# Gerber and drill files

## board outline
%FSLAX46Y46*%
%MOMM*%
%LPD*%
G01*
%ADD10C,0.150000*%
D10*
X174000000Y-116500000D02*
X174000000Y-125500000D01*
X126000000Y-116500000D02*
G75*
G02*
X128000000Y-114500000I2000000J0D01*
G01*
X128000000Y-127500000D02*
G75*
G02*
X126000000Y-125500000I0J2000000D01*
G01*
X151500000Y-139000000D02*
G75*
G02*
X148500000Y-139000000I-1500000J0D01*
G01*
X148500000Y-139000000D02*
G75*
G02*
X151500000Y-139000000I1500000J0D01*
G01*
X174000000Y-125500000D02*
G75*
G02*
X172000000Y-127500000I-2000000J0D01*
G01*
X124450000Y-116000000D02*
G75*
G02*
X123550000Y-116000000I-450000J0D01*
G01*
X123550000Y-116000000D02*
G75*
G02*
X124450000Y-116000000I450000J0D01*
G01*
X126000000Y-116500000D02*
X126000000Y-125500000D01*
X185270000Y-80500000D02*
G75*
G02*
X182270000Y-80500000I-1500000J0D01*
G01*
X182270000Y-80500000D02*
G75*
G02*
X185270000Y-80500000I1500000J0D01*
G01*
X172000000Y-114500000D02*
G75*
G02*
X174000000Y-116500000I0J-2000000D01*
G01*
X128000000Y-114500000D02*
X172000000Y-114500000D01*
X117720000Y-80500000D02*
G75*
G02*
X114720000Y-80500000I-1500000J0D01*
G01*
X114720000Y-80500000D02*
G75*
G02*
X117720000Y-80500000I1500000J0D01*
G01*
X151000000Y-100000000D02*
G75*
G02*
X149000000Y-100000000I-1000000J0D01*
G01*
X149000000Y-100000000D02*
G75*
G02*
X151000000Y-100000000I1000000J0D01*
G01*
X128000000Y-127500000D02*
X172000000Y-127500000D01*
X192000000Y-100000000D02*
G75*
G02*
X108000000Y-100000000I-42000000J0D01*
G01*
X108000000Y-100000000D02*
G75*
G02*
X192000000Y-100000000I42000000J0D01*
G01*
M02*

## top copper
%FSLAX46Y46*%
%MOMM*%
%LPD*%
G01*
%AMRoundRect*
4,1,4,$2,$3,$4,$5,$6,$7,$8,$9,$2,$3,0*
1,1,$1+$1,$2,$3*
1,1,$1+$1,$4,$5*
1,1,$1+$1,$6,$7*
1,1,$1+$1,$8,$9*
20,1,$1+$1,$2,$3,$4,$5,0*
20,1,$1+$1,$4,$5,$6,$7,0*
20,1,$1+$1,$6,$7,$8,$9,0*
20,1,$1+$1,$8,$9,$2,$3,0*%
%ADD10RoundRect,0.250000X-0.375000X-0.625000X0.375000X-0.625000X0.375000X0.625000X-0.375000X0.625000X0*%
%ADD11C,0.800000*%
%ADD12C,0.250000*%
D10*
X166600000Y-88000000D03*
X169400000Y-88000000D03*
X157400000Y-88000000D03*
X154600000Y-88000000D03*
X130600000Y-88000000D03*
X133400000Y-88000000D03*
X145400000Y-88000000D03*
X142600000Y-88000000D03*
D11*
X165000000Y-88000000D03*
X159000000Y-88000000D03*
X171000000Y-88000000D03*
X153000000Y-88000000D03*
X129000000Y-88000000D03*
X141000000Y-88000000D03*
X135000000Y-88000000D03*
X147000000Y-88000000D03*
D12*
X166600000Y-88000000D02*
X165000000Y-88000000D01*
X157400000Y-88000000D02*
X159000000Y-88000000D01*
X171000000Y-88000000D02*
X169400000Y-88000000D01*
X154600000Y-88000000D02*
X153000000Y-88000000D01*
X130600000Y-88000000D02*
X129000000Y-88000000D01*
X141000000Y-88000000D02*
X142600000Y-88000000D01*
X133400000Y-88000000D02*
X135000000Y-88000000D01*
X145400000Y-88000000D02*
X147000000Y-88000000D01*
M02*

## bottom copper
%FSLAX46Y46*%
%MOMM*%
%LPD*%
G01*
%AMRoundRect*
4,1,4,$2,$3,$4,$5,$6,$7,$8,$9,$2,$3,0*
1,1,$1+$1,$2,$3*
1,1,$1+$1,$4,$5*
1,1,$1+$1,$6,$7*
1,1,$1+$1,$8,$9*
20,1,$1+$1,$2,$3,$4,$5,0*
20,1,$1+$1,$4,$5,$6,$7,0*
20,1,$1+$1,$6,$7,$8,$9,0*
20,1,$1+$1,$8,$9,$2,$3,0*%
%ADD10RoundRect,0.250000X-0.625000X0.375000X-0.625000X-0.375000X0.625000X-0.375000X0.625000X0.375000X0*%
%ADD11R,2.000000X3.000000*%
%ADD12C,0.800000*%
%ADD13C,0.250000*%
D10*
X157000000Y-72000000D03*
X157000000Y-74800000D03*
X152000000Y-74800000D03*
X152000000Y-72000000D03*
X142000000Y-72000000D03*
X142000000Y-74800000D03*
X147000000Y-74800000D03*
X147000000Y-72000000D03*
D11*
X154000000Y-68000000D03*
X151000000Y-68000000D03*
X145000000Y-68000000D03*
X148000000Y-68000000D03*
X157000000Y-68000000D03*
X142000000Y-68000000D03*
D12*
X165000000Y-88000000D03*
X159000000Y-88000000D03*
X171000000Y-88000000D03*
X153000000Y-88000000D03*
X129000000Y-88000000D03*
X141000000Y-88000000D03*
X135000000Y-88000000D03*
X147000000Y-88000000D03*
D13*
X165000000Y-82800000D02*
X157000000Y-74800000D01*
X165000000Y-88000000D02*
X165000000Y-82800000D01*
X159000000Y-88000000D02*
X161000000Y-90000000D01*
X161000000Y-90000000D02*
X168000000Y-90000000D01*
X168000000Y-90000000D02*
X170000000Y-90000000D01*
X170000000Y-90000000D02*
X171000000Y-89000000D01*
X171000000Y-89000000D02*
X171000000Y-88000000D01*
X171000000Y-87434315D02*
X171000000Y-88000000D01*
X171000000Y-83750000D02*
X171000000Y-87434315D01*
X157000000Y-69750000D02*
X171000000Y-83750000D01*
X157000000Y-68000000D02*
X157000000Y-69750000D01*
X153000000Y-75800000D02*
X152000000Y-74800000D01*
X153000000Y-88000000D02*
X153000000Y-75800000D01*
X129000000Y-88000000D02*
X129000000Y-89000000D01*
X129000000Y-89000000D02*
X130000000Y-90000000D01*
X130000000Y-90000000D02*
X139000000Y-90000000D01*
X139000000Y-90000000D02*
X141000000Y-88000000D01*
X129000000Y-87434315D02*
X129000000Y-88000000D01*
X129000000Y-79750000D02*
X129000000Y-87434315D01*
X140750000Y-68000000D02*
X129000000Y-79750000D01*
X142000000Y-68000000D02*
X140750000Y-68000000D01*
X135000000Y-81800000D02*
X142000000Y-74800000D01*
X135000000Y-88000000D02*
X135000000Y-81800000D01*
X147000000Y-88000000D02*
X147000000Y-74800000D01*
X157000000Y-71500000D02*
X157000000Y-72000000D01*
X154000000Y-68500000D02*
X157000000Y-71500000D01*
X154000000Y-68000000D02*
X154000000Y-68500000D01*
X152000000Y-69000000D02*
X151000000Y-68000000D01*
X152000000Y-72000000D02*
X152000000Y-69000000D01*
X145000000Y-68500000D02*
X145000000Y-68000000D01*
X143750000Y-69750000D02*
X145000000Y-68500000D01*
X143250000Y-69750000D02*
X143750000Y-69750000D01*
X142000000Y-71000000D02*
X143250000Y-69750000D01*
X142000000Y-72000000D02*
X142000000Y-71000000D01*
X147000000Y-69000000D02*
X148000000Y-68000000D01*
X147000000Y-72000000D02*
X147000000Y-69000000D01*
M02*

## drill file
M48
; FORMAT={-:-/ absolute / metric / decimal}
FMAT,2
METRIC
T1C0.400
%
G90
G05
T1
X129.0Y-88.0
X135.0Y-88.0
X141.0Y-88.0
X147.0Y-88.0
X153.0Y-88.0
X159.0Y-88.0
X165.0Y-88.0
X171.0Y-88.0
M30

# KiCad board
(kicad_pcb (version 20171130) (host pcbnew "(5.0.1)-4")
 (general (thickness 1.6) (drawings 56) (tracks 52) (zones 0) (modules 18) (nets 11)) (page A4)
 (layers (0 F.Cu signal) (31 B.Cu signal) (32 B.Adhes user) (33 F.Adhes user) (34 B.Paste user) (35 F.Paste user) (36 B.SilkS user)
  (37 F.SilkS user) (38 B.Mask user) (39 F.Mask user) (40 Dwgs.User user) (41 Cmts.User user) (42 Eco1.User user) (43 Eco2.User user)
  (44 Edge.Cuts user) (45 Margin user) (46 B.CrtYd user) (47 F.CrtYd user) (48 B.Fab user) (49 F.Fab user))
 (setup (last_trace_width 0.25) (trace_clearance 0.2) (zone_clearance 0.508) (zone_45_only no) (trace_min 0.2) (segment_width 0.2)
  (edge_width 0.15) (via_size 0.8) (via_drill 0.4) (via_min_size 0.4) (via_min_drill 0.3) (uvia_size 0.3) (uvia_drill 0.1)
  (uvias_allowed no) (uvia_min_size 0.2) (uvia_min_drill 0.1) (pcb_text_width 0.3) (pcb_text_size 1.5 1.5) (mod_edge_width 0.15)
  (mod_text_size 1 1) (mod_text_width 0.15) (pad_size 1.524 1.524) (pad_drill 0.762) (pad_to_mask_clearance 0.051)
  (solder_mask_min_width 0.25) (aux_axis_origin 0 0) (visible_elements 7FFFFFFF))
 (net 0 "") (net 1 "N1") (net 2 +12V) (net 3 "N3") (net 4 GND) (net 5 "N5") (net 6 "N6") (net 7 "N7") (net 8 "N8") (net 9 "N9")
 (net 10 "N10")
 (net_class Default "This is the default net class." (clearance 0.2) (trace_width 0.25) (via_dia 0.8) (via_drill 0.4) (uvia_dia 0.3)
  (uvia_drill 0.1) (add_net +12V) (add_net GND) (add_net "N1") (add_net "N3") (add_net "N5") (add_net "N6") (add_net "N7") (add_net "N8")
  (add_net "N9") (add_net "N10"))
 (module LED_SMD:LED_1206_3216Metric (layer F.Cu) (at 168 88)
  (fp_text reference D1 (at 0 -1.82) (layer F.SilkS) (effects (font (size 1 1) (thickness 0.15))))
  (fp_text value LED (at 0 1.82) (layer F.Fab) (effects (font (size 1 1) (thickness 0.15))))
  (pad 1 smd roundrect (at -1.4 0) (size 1.25 1.75) (layers F.Cu F.Paste F.Mask) (roundrect_rratio 0.2) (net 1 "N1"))
  (pad 2 smd roundrect (at 1.4 0) (size 1.25 1.75) (layers F.Cu F.Paste F.Mask) (roundrect_rratio 0.2) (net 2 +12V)))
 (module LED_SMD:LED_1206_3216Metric (layer F.Cu) (at 156 88)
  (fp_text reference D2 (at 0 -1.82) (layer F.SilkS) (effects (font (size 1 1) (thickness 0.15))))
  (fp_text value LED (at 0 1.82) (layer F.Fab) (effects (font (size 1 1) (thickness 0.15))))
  (pad 2 smd roundrect (at 1.4 0) (size 1.25 1.75) (layers F.Cu F.Paste F.Mask) (roundrect_rratio 0.2) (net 2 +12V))
  (pad 1 smd roundrect (at -1.4 0) (size 1.25 1.75) (layers F.Cu F.Paste F.Mask) (roundrect_rratio 0.2) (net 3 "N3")))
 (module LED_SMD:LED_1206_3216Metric (layer F.Cu) (at 132 88)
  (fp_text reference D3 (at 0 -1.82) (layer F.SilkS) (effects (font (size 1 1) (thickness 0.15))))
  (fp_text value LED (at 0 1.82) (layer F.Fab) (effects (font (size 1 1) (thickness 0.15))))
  (pad 1 smd roundrect (at -1.4 0) (size 1.25 1.75) (layers F.Cu F.Paste F.Mask) (roundrect_rratio 0.2) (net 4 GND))
  (pad 2 smd roundrect (at 1.4 0) (size 1.25 1.75) (layers F.Cu F.Paste F.Mask) (roundrect_rratio 0.2) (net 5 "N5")))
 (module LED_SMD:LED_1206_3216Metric (layer F.Cu) (at 144 88)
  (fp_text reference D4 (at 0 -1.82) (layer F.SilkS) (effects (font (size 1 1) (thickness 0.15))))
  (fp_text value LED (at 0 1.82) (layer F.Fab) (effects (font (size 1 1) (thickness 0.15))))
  (pad 2 smd roundrect (at 1.4 0) (size 1.25 1.75) (layers F.Cu F.Paste F.Mask) (roundrect_rratio 0.2) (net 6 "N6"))
  (pad 1 smd roundrect (at -1.4 0) (size 1.25 1.75) (layers F.Cu F.Paste F.Mask) (roundrect_rratio 0.2) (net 4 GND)))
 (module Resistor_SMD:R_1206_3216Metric (layer B.Cu) (at 157 73.4 270)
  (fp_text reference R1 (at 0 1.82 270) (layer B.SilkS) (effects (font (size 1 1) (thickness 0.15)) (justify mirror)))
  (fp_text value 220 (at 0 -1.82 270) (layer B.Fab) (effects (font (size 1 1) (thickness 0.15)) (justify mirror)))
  (pad 1 smd roundrect (at -1.4 0 270) (size 1.25 1.75) (layers B.Cu B.Paste B.Mask) (roundrect_rratio 0.2) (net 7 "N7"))
  (pad 2 smd roundrect (at 1.4 0 270) (size 1.25 1.75) (layers B.Cu B.Paste B.Mask) (roundrect_rratio 0.2) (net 1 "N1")))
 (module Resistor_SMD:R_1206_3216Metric (layer B.Cu) (at 152 73.4 270)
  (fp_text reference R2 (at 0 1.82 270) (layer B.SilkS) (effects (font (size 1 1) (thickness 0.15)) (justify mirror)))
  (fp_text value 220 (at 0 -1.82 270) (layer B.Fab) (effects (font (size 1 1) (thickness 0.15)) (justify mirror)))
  (pad 2 smd roundrect (at 1.4 0 270) (size 1.25 1.75) (layers B.Cu B.Paste B.Mask) (roundrect_rratio 0.2) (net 3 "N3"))
  (pad 1 smd roundrect (at -1.4 0 270) (size 1.25 1.75) (layers B.Cu B.Paste B.Mask) (roundrect_rratio 0.2) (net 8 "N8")))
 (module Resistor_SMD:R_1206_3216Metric (layer B.Cu) (at 142 73.4 270)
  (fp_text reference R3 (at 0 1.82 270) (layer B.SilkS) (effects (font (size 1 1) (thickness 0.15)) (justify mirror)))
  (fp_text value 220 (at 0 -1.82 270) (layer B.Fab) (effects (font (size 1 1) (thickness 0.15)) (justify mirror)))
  (pad 1 smd roundrect (at -1.4 0 270) (size 1.25 1.75) (layers B.Cu B.Paste B.Mask) (roundrect_rratio 0.2) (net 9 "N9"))
  (pad 2 smd roundrect (at 1.4 0 270) (size 1.25 1.75) (layers B.Cu B.Paste B.Mask) (roundrect_rratio 0.2) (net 5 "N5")))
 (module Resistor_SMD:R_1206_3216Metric (layer B.Cu) (at 147 73.4 270)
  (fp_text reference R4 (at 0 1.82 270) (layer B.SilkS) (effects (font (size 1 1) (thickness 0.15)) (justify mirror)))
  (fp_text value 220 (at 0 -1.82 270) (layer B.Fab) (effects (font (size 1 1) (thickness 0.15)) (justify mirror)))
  (pad 2 smd roundrect (at 1.4 0 270) (size 1.25 1.75) (layers B.Cu B.Paste B.Mask) (roundrect_rratio 0.2) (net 6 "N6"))
  (pad 1 smd roundrect (at -1.4 0 270) (size 1.25 1.75) (layers B.Cu B.Paste B.Mask) (roundrect_rratio 0.2) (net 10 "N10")))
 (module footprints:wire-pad (layer B.Cu) (at 154 66)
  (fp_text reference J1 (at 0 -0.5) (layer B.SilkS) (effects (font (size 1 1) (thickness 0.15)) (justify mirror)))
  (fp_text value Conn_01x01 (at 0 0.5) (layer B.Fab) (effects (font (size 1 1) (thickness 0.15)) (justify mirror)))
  (pad 1 smd rect (at 0 2) (size 2 3) (layers B.Cu B.Paste B.Mask) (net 7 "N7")))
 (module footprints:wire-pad (layer B.Cu) (at 151 66)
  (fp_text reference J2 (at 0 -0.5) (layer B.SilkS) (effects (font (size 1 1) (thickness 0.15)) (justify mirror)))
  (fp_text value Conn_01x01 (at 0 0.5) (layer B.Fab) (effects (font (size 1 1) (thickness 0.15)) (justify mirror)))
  (pad 1 smd rect (at 0 2) (size 2 3) (layers B.Cu B.Paste B.Mask) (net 8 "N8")))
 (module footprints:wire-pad (layer B.Cu) (at 145 66)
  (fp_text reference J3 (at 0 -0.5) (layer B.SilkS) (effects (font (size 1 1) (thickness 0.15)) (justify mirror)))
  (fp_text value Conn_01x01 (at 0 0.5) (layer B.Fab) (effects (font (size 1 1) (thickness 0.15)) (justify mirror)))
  (pad 1 smd rect (at 0 2) (size 2 3) (layers B.Cu B.Paste B.Mask) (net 9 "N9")))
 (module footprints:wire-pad (layer B.Cu) (at 148 66)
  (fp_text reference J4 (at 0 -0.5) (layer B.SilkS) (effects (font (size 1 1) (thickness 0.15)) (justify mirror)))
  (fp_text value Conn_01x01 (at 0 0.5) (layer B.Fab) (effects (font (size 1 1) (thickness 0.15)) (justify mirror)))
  (pad 1 smd rect (at 0 2) (size 2 3) (layers B.Cu B.Paste B.Mask) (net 10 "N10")))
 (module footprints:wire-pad (layer B.Cu) (at 157 66)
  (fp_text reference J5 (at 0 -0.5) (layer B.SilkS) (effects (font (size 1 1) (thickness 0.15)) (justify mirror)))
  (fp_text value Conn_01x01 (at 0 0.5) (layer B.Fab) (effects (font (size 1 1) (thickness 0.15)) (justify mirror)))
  (pad 1 smd rect (at 0 2) (size 2 3) (layers B.Cu B.Paste B.Mask) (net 2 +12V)))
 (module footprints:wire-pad (layer B.Cu) (at 142 66)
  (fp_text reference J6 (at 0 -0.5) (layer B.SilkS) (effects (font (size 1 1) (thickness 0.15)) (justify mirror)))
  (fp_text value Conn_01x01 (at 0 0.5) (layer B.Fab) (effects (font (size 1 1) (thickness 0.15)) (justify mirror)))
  (pad 1 smd rect (at 0 2) (size 2 3) (layers B.Cu B.Paste B.Mask) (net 4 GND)))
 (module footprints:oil (layer F.Cu) (at 168 92)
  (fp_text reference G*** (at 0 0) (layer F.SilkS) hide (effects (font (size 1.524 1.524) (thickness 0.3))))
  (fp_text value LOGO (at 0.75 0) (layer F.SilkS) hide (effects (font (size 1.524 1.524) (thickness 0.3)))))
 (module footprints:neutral (layer F.Cu) (at 156 92)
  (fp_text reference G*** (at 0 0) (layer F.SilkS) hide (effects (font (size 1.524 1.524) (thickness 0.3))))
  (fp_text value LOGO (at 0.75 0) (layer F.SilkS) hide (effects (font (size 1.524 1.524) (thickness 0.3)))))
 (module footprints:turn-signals (layer F.Cu) (at 144 92)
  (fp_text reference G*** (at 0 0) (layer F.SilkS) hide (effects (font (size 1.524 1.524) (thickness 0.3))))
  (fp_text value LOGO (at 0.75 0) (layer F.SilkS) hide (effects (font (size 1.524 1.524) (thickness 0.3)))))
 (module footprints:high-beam (layer F.Cu) (at 132 92)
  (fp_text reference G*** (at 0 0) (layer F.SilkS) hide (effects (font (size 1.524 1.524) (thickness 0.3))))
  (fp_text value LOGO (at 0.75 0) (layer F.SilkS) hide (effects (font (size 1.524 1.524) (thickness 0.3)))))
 (gr_line (start 174 116.5) (end 174 125.5) (layer Edge.Cuts) (width 0.15))
 (gr_arc (start 128 116.5) (end 128 114.5) (angle -90) (layer Edge.Cuts) (width 0.15))
 (gr_arc (start 128 125.5) (end 126 125.5) (angle -90) (layer Edge.Cuts) (width 0.15))
 (gr_circle (center 150 139) (end 151.5 139) (layer Edge.Cuts) (width 0.15))
 (gr_arc (start 172 125.5) (end 172 127.5) (angle -90) (layer Edge.Cuts) (width 0.15))
 (gr_circle (center 124 116) (end 124.45 116) (layer Edge.Cuts) (width 0.15))
 (gr_line (start 126 116.5) (end 126 125.5) (layer Edge.Cuts) (width 0.15))
 (gr_circle (center 183.77 80.5) (end 185.27 80.5) (layer Edge.Cuts) (width 0.15))
 (gr_arc (start 172 116.5) (end 174 116.5) (angle -90) (layer Edge.Cuts) (width 0.15))
 (gr_line (start 128 114.5) (end 172 114.5) (layer Edge.Cuts) (width 0.15))
 (gr_circle (center 116.22 80.5) (end 117.72 80.5) (layer Edge.Cuts) (width 0.15))
 (gr_circle (center 150 100) (end 151 100) (layer Edge.Cuts) (width 0.15))
 (gr_line (start 128 127.5) (end 172 127.5) (layer Edge.Cuts) (width 0.15))
 (gr_circle (center 150 100) (end 192 100) (layer Edge.Cuts) (width 0.15))
 (via (at 165 88) (size 0.8) (drill 0.4) (layers F.Cu B.Cu) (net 1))
 (segment (start 166.6 88) (end 165 88) (width 0.25) (layer F.Cu) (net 1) (status 10))
 (segment (start 165 82.8) (end 157 74.8) (width 0.25) (layer B.Cu) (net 1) (status 20))
 (segment (start 165 88) (end 165 82.8) (width 0.25) (layer B.Cu) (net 1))
 (via (at 159 88) (size 0.8) (drill 0.4) (layers F.Cu B.Cu) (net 2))
 (segment (start 157.4 88) (end 159 88) (width 0.25) (layer F.Cu) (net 2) (status 10))
 (segment (start 159 88) (end 161 90) (width 0.25) (layer B.Cu) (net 2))
 (segment (start 161 90) (end 168 90) (width 0.25) (layer B.Cu) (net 2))
 (segment (start 168 90) (end 170 90) (width 0.25) (layer B.Cu) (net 2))
 (segment (start 170 90) (end 171 89) (width 0.25) (layer B.Cu) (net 2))
 (via (at 171 88) (size 0.8) (drill 0.4) (layers F.Cu B.Cu) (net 2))
 (segment (start 171 89) (end 171 88) (width 0.25) (layer B.Cu) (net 2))
 (segment (start 171 88) (end 169.4 88) (width 0.25) (layer F.Cu) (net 2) (status 20))
 (segment (start 171 87.434315) (end 171 88) (width 0.25) (layer B.Cu) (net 2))
 (segment (start 171 83.75) (end 171 87.434315) (width 0.25) (layer B.Cu) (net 2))
 (segment (start 157 69.75) (end 171 83.75) (width 0.25) (layer B.Cu) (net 2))
 (segment (start 157 68) (end 157 69.75) (width 0.25) (layer B.Cu) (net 2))
 (via (at 153 88) (size 0.8) (drill 0.4) (layers F.Cu B.Cu) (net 3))
 (segment (start 154.6 88) (end 153 88) (width 0.25) (layer F.Cu) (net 3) (status 10))
 (segment (start 153 75.8) (end 152 74.8) (width 0.25) (layer B.Cu) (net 3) (status 20))
 (segment (start 153 88) (end 153 75.8) (width 0.25) (layer B.Cu) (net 3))
 (via (at 129 88) (size 0.8) (drill 0.4) (layers F.Cu B.Cu) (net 4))
 (segment (start 130.6 88) (end 129 88) (width 0.25) (layer F.Cu) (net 4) (status 10))
 (segment (start 129 88) (end 129 89) (width 0.25) (layer B.Cu) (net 4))
 (segment (start 129 89) (end 130 90) (width 0.25) (layer B.Cu) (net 4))
 (via (at 141 88) (size 0.8) (drill 0.4) (layers F.Cu B.Cu) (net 4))
 (segment (start 130 90) (end 139 90) (width 0.25) (layer B.Cu) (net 4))
 (segment (start 139 90) (end 141 88) (width 0.25) (layer B.Cu) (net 4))
 (segment (start 141 88) (end 142.6 88) (width 0.25) (layer F.Cu) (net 4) (status 20))
 (segment (start 129 87.434315) (end 129 88) (width 0.25) (layer B.Cu) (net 4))
 (segment (start 129 79.75) (end 129 87.434315) (width 0.25) (layer B.Cu) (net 4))
 (segment (start 140.75 68) (end 129 79.75) (width 0.25) (layer B.Cu) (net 4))
 (segment (start 142 68) (end 140.75 68) (width 0.25) (layer B.Cu) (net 4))
 (via (at 135 88) (size 0.8) (drill 0.4) (layers F.Cu B.Cu) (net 5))
 (segment (start 133.4 88) (end 135 88) (width 0.25) (layer F.Cu) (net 5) (status 10))
 (segment (start 135 81.8) (end 142 74.8) (width 0.25) (layer B.Cu) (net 5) (status 20))
 (segment (start 135 88) (end 135 81.8) (width 0.25) (layer B.Cu) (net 5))
 (via (at 147 88) (size 0.8) (drill 0.4) (layers F.Cu B.Cu) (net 6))
 (segment (start 145.4 88) (end 147 88) (width 0.25) (layer F.Cu) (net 6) (status 10))
 (segment (start 147 88) (end 147 74.8) (width 0.25) (layer B.Cu) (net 6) (status 20))
 (segment (start 157 71.5) (end 157 72) (width 0.25) (layer B.Cu) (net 7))
 (segment (start 154 68.5) (end 157 71.5) (width 0.25) (layer B.Cu) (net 7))
 (segment (start 154 68) (end 154 68.5) (width 0.25) (layer B.Cu) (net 7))
 (segment (start 152 69) (end 151 68) (width 0.25) (layer B.Cu) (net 8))
 (segment (start 152 72) (end 152 69) (width 0.25) (layer B.Cu) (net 8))
 (segment (start 145 68.5) (end 145 68) (width 0.25) (layer B.Cu) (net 9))
 (segment (start 143.75 69.75) (end 145 68.5) (width 0.25) (layer B.Cu) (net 9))
 (segment (start 143.25 69.75) (end 143.75 69.75) (width 0.25) (layer B.Cu) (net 9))
 (segment (start 142 71) (end 143.25 69.75) (width 0.25) (layer B.Cu) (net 9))
 (segment (start 142 72) (end 142 71) (width 0.25) (layer B.Cu) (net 9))
 (segment (start 147 69) (end 148 68) (width 0.25) (layer B.Cu) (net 10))
 (segment (start 147 72) (end 147 69) (width 0.25) (layer B.Cu) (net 10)))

